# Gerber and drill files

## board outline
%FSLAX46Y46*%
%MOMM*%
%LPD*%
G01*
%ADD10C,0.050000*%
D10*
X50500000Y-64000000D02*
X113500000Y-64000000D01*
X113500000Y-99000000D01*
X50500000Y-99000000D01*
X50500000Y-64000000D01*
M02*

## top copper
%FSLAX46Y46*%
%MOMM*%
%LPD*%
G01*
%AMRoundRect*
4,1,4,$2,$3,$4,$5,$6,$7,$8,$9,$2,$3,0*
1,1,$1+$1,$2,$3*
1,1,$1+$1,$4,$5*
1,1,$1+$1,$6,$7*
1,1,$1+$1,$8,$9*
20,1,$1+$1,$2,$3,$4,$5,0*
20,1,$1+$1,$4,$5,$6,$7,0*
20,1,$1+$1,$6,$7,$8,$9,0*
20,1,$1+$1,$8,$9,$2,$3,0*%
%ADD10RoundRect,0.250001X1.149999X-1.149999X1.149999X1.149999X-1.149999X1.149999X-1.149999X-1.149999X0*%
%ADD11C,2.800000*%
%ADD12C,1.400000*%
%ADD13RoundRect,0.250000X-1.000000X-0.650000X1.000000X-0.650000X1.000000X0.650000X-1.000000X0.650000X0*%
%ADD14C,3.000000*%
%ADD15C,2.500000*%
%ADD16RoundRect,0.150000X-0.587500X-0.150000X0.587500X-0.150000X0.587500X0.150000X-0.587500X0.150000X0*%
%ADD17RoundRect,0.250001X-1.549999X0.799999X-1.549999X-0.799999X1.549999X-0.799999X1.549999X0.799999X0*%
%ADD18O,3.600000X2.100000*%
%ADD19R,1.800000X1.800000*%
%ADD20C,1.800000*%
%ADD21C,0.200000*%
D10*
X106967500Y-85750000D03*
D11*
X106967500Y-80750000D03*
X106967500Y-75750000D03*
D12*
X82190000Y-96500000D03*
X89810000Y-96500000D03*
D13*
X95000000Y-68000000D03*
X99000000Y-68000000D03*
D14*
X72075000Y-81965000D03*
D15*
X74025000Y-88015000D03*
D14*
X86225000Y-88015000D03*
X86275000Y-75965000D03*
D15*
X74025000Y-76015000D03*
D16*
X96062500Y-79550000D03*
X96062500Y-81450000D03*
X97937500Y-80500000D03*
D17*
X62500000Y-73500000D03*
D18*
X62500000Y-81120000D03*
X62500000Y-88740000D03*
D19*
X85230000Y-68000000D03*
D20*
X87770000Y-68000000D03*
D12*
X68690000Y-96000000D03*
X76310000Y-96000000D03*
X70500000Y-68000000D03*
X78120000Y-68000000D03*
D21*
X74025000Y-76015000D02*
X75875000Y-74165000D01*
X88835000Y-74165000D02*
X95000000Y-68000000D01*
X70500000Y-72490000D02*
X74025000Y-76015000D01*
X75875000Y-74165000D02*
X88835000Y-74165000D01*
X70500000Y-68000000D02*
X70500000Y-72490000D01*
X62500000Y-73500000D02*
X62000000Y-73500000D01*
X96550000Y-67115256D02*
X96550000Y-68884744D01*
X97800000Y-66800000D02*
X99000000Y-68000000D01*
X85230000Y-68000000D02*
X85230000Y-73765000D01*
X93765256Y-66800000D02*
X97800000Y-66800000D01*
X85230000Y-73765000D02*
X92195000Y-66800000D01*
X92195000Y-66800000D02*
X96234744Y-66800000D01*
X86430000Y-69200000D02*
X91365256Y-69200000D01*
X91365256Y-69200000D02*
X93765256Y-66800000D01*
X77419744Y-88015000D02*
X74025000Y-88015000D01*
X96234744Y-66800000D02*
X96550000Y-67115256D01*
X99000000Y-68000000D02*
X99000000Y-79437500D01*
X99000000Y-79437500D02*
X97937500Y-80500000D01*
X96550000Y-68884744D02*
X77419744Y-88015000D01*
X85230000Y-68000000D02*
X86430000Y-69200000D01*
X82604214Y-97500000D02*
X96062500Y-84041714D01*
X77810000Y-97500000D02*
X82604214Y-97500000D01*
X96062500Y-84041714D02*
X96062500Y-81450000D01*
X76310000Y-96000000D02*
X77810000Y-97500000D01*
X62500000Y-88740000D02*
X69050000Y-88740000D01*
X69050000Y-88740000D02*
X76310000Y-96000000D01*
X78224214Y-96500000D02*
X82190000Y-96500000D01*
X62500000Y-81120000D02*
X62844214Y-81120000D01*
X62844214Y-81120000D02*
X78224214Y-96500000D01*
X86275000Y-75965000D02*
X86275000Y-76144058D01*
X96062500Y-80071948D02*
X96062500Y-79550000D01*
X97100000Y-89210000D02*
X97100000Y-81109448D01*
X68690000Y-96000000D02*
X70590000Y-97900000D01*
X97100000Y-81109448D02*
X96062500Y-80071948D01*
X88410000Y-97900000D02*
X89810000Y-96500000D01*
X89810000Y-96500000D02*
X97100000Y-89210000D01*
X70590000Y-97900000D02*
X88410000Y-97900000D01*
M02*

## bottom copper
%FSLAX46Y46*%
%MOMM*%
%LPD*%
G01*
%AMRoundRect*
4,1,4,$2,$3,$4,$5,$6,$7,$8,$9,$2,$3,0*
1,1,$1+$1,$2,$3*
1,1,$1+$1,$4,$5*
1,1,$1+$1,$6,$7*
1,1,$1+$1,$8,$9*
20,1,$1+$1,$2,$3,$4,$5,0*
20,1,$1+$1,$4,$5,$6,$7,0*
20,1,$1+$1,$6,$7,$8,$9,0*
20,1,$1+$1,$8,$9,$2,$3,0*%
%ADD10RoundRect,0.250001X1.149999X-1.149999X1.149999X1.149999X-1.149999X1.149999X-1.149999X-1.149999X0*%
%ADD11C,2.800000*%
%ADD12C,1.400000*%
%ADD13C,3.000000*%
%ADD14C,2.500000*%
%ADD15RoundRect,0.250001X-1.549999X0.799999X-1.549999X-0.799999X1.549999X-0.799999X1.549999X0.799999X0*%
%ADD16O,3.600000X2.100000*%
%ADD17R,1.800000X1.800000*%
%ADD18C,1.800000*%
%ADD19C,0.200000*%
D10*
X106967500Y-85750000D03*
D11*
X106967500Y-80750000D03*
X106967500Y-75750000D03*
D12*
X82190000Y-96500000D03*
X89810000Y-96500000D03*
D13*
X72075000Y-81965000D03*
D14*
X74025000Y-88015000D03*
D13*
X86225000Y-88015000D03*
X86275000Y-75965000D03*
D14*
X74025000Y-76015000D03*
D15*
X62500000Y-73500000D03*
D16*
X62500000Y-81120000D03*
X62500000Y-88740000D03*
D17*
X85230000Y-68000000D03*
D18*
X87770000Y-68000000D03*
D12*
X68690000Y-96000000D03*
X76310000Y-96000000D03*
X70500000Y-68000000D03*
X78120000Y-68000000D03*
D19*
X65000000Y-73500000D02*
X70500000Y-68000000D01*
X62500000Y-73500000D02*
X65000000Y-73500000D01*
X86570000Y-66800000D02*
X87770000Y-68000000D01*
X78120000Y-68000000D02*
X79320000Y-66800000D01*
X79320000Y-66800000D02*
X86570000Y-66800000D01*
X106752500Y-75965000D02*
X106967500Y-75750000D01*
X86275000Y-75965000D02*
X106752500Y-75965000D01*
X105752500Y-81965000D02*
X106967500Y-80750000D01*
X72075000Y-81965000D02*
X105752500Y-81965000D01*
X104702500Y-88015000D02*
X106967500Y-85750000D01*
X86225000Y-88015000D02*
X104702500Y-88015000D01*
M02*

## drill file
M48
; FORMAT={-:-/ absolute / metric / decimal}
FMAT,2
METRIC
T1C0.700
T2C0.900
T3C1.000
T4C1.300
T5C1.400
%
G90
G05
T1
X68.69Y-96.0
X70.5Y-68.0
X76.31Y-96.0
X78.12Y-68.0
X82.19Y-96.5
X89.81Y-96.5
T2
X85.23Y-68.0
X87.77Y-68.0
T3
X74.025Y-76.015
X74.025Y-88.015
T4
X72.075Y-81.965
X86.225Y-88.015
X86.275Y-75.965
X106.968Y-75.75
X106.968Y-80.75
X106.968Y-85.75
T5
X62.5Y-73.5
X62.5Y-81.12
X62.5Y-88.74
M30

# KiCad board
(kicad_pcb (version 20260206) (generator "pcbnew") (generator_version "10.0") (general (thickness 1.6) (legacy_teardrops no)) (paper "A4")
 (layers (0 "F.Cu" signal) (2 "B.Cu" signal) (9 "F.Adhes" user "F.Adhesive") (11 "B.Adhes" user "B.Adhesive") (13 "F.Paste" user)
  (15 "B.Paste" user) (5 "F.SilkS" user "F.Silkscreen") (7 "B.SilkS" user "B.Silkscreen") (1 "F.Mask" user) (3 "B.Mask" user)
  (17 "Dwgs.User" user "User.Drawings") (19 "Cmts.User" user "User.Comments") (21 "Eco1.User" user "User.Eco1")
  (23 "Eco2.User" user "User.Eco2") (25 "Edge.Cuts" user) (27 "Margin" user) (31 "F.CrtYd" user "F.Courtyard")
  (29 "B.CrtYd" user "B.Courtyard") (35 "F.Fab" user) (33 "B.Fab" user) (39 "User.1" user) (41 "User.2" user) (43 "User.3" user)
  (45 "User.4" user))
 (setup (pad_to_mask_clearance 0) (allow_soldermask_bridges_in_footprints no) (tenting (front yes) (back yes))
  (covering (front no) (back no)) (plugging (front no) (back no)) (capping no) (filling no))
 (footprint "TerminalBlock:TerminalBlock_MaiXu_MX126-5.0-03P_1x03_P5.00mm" (layer "F.Cu") (at 106.9675 85.75 90)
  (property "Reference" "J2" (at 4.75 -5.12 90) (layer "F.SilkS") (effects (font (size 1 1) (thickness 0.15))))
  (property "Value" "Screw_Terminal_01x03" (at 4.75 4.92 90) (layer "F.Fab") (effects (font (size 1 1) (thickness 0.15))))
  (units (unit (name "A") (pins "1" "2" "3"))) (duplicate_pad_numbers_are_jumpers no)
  (pad "1" thru_hole roundrect (at 0 0 90) (size 2.8 2.8) (drill 1.3) (layers "*.Cu" "*.Mask") (remove_unused_layers no)
   (roundrect_rratio 0.089286) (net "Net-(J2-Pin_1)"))
  (pad "2" thru_hole circle (at 5 0 90) (size 2.8 2.8) (drill 1.3) (layers "*.Cu" "*.Mask") (remove_unused_layers no) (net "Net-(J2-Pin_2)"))
  (pad "3" thru_hole circle (at 10 0 90) (size 2.8 2.8) (drill 1.3) (layers "*.Cu" "*.Mask") (remove_unused_layers no)
   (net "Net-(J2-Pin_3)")))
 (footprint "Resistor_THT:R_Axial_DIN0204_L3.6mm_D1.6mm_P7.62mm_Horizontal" (layer "F.Cu") (at 82.19 96.5)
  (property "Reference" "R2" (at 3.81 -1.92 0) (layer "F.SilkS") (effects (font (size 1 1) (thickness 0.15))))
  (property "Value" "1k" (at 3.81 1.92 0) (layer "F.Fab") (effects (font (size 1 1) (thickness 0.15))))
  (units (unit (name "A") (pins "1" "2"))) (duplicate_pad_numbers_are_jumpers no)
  (pad "1" thru_hole circle (at 0 0) (size 1.4 1.4) (drill 0.7) (layers "*.Cu" "*.Mask") (remove_unused_layers no) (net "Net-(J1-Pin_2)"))
  (pad "2" thru_hole circle (at 7.62 0) (size 1.4 1.4) (drill 0.7) (layers "*.Cu" "*.Mask") (remove_unused_layers no) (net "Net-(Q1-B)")))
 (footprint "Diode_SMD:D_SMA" (layer "F.Cu") (at 97 68)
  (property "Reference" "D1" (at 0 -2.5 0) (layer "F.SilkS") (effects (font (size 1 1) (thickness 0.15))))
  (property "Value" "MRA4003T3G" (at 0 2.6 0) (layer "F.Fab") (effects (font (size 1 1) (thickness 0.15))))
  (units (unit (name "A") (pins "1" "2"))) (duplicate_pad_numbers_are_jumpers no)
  (pad "1" smd roundrect (at -2 0) (size 2.5 1.8) (layers "F.Cu" "F.Mask" "F.Paste") (roundrect_rratio 0.1388888889) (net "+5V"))
  (pad "2" smd roundrect (at 2 0) (size 2.5 1.8) (layers "F.Cu" "F.Mask" "F.Paste") (roundrect_rratio 0.1388888889) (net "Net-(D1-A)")))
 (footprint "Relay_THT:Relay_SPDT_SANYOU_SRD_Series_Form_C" (layer "F.Cu") (at 72.075 81.965)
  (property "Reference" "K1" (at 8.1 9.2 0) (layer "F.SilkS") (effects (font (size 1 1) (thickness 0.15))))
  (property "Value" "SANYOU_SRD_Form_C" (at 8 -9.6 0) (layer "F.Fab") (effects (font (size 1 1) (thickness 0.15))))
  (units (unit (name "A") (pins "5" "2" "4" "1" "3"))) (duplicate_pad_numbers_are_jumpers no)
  (pad "1" thru_hole circle (at 0 0 90) (size 3 3) (drill 1.3) (layers "*.Cu" "*.Mask") (remove_unused_layers no) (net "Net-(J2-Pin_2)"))
  (pad "2" thru_hole circle (at 1.95 6.05 90) (size 2.5 2.5) (drill 1) (layers "*.Cu" "*.Mask") (remove_unused_layers no) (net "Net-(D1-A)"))
  (pad "3" thru_hole circle (at 14.15 6.05 90) (size 3 3) (drill 1.3) (layers "*.Cu" "*.Mask") (remove_unused_layers no)
   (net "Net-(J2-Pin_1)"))
  (pad "4" thru_hole circle (at 14.2 -6 90) (size 3 3) (drill 1.3) (layers "*.Cu" "*.Mask") (remove_unused_layers no) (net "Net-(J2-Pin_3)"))
  (pad "5" thru_hole circle (at 1.95 -5.95 90) (size 2.5 2.5) (drill 1) (layers "*.Cu" "*.Mask") (remove_unused_layers no) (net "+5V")))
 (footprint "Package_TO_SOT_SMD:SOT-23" (layer "F.Cu") (at 97 80.5)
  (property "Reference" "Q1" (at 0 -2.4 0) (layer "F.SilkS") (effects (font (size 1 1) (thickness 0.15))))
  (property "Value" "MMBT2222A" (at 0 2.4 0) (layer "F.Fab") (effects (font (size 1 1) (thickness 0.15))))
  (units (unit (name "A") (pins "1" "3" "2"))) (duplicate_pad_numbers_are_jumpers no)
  (pad "1" smd roundrect (at -0.9375 -0.95) (size 1.475 0.6) (layers "F.Cu" "F.Mask" "F.Paste") (roundrect_rratio 0.25) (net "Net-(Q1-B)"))
  (pad "2" smd roundrect (at -0.9375 0.95) (size 1.475 0.6) (layers "F.Cu" "F.Mask" "F.Paste") (roundrect_rratio 0.25) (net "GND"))
  (pad "3" smd roundrect (at 0.9375 0) (size 1.475 0.6) (layers "F.Cu" "F.Mask" "F.Paste") (roundrect_rratio 0.25) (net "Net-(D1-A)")))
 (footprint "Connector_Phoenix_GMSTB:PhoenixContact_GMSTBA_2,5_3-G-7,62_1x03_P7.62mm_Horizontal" (layer "F.Cu") (at 62.5 73.5 -90)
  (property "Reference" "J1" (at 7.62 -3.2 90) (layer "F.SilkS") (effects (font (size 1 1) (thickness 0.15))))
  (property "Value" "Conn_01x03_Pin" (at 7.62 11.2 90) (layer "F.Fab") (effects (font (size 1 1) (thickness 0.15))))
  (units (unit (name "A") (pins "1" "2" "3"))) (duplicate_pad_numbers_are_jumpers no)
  (pad "1" thru_hole roundrect (at 0 0 270) (size 2.1 3.6) (drill 1.4) (layers "*.Cu" "*.Mask") (remove_unused_layers no)
   (roundrect_rratio 0.119048) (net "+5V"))
  (pad "2" thru_hole oval (at 7.62 0 270) (size 2.1 3.6) (drill 1.4) (layers "*.Cu" "*.Mask") (remove_unused_layers no)
   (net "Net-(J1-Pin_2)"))
  (pad "3" thru_hole oval (at 15.24 0 270) (size 2.1 3.6) (drill 1.4) (layers "*.Cu" "*.Mask") (remove_unused_layers no) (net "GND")))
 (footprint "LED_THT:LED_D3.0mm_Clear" (layer "F.Cu") (at 85.23 68)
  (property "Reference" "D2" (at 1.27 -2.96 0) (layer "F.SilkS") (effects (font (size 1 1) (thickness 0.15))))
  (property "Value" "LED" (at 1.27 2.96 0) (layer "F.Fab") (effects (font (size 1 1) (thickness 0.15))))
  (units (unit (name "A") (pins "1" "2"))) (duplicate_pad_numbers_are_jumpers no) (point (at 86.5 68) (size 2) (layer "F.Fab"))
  (pad "1" thru_hole rect (at 0 0) (size 1.8 1.8) (drill 0.9) (layers "*.Cu" "*.Mask") (remove_unused_layers no) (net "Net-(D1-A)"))
  (pad "2" thru_hole circle (at 2.54 0) (size 1.8 1.8) (drill 0.9) (layers "*.Cu" "*.Mask") (remove_unused_layers no) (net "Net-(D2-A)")))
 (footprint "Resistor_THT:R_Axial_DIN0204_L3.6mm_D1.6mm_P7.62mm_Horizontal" (layer "F.Cu") (at 68.69 96)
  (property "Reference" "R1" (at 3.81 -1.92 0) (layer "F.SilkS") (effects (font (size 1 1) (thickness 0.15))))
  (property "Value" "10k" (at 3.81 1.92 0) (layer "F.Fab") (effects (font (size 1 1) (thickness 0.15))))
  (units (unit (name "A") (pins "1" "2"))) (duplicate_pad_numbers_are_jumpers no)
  (pad "1" thru_hole circle (at 0 0) (size 1.4 1.4) (drill 0.7) (layers "*.Cu" "*.Mask") (remove_unused_layers no) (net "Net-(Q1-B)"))
  (pad "2" thru_hole circle (at 7.62 0) (size 1.4 1.4) (drill 0.7) (layers "*.Cu" "*.Mask") (remove_unused_layers no) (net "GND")))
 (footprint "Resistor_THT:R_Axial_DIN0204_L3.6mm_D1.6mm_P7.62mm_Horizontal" (layer "F.Cu") (at 70.5 68)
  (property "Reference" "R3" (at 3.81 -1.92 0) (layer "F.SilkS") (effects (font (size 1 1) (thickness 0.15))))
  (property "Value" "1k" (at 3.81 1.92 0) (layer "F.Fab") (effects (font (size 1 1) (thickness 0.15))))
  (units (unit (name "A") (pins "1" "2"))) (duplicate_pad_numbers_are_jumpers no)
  (pad "1" thru_hole circle (at 0 0) (size 1.4 1.4) (drill 0.7) (layers "*.Cu" "*.Mask") (remove_unused_layers no) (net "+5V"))
  (pad "2" thru_hole circle (at 7.62 0) (size 1.4 1.4) (drill 0.7) (layers "*.Cu" "*.Mask") (remove_unused_layers no) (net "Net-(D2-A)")))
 (gr_rect (start 50.5 64) (end 113.5 99) (stroke (width 0.05) (type default)) (fill no) (layer "Edge.Cuts"))
 (segment (start 74.025 76.015) (end 75.875 74.165) (width 0.2) (layer "F.Cu") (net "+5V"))
 (segment (start 88.835 74.165) (end 95 68) (width 0.2) (layer "F.Cu") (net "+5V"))
 (segment (start 70.5 72.49) (end 74.025 76.015) (width 0.2) (layer "F.Cu") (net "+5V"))
 (segment (start 75.875 74.165) (end 88.835 74.165) (width 0.2) (layer "F.Cu") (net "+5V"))
 (segment (start 70.5 68) (end 70.5 72.49) (width 0.2) (layer "F.Cu") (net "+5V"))
 (segment (start 62.5 73.5) (end 62 73.5) (width 0.2) (layer "F.Cu") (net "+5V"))
 (segment (start 65 73.5) (end 70.5 68) (width 0.2) (layer "B.Cu") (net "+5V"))
 (segment (start 62.5 73.5) (end 65 73.5) (width 0.2) (layer "B.Cu") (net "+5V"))
 (segment (start 96.55 67.115256) (end 96.55 68.884744) (width 0.2) (layer "F.Cu") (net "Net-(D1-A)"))
 (segment (start 97.8 66.8) (end 99 68) (width 0.2) (layer "F.Cu") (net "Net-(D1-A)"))
 (segment (start 85.23 68) (end 85.23 73.765) (width 0.2) (layer "F.Cu") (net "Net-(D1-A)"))
 (segment (start 93.765256 66.8) (end 97.8 66.8) (width 0.2) (layer "F.Cu") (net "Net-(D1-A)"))
 (segment (start 85.23 73.765) (end 92.195 66.8) (width 0.2) (layer "F.Cu") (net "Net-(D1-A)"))
 (segment (start 92.195 66.8) (end 96.234744 66.8) (width 0.2) (layer "F.Cu") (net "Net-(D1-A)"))
 (segment (start 86.43 69.2) (end 91.365256 69.2) (width 0.2) (layer "F.Cu") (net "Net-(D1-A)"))
 (segment (start 91.365256 69.2) (end 93.765256 66.8) (width 0.2) (layer "F.Cu") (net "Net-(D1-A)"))
 (segment (start 77.419744 88.015) (end 74.025 88.015) (width 0.2) (layer "F.Cu") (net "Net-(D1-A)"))
 (segment (start 96.234744 66.8) (end 96.55 67.115256) (width 0.2) (layer "F.Cu") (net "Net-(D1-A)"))
 (segment (start 99 68) (end 99 79.4375) (width 0.2) (layer "F.Cu") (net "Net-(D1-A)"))
 (segment (start 99 79.4375) (end 97.9375 80.5) (width 0.2) (layer "F.Cu") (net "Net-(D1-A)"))
 (segment (start 96.55 68.884744) (end 77.419744 88.015) (width 0.2) (layer "F.Cu") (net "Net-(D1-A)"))
 (segment (start 85.23 68) (end 86.43 69.2) (width 0.2) (layer "F.Cu") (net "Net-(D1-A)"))
 (segment (start 86.57 66.8) (end 87.77 68) (width 0.2) (layer "B.Cu") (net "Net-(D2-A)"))
 (segment (start 78.12 68) (end 79.32 66.8) (width 0.2) (layer "B.Cu") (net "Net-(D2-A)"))
 (segment (start 79.32 66.8) (end 86.57 66.8) (width 0.2) (layer "B.Cu") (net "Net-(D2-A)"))
 (segment (start 82.604214 97.5) (end 96.0625 84.041714) (width 0.2) (layer "F.Cu") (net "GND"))
 (segment (start 77.81 97.5) (end 82.604214 97.5) (width 0.2) (layer "F.Cu") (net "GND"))
 (segment (start 96.0625 84.041714) (end 96.0625 81.45) (width 0.2) (layer "F.Cu") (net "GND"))
 (segment (start 76.31 96) (end 77.81 97.5) (width 0.2) (layer "F.Cu") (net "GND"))
 (segment (start 62.5 88.74) (end 69.05 88.74) (width 0.2) (layer "F.Cu") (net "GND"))
 (segment (start 69.05 88.74) (end 76.31 96) (width 0.2) (layer "F.Cu") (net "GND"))
 (segment (start 78.224214 96.5) (end 82.19 96.5) (width 0.2) (layer "F.Cu") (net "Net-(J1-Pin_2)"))
 (segment (start 62.5 81.12) (end 62.844214 81.12) (width 0.2) (layer "F.Cu") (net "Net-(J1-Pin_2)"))
 (segment (start 62.844214 81.12) (end 78.224214 96.5) (width 0.2) (layer "F.Cu") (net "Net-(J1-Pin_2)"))
 (segment (start 86.275 75.965) (end 86.275 76.144058) (width 0.2) (layer "F.Cu") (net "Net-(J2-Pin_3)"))
 (segment (start 106.7525 75.965) (end 106.9675 75.75) (width 0.2) (layer "B.Cu") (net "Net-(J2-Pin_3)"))
 (segment (start 86.275 75.965) (end 106.7525 75.965) (width 0.2) (layer "B.Cu") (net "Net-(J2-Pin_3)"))
 (segment (start 105.7525 81.965) (end 106.9675 80.75) (width 0.2) (layer "B.Cu") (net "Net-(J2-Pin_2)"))
 (segment (start 72.075 81.965) (end 105.7525 81.965) (width 0.2) (layer "B.Cu") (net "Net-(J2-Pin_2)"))
 (segment (start 104.7025 88.015) (end 106.9675 85.75) (width 0.2) (layer "B.Cu") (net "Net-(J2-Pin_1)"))
 (segment (start 86.225 88.015) (end 104.7025 88.015) (width 0.2) (layer "B.Cu") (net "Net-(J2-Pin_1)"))
 (segment (start 96.0625 80.071948) (end 96.0625 79.55) (width 0.2) (layer "F.Cu") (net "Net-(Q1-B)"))
 (segment (start 97.1 89.21) (end 97.1 81.109448) (width 0.2) (layer "F.Cu") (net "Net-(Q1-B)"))
 (segment (start 68.69 96) (end 70.59 97.9) (width 0.2) (layer "F.Cu") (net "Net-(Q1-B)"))
 (segment (start 97.1 81.109448) (end 96.0625 80.071948) (width 0.2) (layer "F.Cu") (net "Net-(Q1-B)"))
 (segment (start 88.41 97.9) (end 89.81 96.5) (width 0.2) (layer "F.Cu") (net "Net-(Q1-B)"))
 (segment (start 89.81 96.5) (end 97.1 89.21) (width 0.2) (layer "F.Cu") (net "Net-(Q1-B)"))
 (segment (start 70.59 97.9) (end 88.41 97.9) (width 0.2) (layer "F.Cu") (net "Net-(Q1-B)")))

